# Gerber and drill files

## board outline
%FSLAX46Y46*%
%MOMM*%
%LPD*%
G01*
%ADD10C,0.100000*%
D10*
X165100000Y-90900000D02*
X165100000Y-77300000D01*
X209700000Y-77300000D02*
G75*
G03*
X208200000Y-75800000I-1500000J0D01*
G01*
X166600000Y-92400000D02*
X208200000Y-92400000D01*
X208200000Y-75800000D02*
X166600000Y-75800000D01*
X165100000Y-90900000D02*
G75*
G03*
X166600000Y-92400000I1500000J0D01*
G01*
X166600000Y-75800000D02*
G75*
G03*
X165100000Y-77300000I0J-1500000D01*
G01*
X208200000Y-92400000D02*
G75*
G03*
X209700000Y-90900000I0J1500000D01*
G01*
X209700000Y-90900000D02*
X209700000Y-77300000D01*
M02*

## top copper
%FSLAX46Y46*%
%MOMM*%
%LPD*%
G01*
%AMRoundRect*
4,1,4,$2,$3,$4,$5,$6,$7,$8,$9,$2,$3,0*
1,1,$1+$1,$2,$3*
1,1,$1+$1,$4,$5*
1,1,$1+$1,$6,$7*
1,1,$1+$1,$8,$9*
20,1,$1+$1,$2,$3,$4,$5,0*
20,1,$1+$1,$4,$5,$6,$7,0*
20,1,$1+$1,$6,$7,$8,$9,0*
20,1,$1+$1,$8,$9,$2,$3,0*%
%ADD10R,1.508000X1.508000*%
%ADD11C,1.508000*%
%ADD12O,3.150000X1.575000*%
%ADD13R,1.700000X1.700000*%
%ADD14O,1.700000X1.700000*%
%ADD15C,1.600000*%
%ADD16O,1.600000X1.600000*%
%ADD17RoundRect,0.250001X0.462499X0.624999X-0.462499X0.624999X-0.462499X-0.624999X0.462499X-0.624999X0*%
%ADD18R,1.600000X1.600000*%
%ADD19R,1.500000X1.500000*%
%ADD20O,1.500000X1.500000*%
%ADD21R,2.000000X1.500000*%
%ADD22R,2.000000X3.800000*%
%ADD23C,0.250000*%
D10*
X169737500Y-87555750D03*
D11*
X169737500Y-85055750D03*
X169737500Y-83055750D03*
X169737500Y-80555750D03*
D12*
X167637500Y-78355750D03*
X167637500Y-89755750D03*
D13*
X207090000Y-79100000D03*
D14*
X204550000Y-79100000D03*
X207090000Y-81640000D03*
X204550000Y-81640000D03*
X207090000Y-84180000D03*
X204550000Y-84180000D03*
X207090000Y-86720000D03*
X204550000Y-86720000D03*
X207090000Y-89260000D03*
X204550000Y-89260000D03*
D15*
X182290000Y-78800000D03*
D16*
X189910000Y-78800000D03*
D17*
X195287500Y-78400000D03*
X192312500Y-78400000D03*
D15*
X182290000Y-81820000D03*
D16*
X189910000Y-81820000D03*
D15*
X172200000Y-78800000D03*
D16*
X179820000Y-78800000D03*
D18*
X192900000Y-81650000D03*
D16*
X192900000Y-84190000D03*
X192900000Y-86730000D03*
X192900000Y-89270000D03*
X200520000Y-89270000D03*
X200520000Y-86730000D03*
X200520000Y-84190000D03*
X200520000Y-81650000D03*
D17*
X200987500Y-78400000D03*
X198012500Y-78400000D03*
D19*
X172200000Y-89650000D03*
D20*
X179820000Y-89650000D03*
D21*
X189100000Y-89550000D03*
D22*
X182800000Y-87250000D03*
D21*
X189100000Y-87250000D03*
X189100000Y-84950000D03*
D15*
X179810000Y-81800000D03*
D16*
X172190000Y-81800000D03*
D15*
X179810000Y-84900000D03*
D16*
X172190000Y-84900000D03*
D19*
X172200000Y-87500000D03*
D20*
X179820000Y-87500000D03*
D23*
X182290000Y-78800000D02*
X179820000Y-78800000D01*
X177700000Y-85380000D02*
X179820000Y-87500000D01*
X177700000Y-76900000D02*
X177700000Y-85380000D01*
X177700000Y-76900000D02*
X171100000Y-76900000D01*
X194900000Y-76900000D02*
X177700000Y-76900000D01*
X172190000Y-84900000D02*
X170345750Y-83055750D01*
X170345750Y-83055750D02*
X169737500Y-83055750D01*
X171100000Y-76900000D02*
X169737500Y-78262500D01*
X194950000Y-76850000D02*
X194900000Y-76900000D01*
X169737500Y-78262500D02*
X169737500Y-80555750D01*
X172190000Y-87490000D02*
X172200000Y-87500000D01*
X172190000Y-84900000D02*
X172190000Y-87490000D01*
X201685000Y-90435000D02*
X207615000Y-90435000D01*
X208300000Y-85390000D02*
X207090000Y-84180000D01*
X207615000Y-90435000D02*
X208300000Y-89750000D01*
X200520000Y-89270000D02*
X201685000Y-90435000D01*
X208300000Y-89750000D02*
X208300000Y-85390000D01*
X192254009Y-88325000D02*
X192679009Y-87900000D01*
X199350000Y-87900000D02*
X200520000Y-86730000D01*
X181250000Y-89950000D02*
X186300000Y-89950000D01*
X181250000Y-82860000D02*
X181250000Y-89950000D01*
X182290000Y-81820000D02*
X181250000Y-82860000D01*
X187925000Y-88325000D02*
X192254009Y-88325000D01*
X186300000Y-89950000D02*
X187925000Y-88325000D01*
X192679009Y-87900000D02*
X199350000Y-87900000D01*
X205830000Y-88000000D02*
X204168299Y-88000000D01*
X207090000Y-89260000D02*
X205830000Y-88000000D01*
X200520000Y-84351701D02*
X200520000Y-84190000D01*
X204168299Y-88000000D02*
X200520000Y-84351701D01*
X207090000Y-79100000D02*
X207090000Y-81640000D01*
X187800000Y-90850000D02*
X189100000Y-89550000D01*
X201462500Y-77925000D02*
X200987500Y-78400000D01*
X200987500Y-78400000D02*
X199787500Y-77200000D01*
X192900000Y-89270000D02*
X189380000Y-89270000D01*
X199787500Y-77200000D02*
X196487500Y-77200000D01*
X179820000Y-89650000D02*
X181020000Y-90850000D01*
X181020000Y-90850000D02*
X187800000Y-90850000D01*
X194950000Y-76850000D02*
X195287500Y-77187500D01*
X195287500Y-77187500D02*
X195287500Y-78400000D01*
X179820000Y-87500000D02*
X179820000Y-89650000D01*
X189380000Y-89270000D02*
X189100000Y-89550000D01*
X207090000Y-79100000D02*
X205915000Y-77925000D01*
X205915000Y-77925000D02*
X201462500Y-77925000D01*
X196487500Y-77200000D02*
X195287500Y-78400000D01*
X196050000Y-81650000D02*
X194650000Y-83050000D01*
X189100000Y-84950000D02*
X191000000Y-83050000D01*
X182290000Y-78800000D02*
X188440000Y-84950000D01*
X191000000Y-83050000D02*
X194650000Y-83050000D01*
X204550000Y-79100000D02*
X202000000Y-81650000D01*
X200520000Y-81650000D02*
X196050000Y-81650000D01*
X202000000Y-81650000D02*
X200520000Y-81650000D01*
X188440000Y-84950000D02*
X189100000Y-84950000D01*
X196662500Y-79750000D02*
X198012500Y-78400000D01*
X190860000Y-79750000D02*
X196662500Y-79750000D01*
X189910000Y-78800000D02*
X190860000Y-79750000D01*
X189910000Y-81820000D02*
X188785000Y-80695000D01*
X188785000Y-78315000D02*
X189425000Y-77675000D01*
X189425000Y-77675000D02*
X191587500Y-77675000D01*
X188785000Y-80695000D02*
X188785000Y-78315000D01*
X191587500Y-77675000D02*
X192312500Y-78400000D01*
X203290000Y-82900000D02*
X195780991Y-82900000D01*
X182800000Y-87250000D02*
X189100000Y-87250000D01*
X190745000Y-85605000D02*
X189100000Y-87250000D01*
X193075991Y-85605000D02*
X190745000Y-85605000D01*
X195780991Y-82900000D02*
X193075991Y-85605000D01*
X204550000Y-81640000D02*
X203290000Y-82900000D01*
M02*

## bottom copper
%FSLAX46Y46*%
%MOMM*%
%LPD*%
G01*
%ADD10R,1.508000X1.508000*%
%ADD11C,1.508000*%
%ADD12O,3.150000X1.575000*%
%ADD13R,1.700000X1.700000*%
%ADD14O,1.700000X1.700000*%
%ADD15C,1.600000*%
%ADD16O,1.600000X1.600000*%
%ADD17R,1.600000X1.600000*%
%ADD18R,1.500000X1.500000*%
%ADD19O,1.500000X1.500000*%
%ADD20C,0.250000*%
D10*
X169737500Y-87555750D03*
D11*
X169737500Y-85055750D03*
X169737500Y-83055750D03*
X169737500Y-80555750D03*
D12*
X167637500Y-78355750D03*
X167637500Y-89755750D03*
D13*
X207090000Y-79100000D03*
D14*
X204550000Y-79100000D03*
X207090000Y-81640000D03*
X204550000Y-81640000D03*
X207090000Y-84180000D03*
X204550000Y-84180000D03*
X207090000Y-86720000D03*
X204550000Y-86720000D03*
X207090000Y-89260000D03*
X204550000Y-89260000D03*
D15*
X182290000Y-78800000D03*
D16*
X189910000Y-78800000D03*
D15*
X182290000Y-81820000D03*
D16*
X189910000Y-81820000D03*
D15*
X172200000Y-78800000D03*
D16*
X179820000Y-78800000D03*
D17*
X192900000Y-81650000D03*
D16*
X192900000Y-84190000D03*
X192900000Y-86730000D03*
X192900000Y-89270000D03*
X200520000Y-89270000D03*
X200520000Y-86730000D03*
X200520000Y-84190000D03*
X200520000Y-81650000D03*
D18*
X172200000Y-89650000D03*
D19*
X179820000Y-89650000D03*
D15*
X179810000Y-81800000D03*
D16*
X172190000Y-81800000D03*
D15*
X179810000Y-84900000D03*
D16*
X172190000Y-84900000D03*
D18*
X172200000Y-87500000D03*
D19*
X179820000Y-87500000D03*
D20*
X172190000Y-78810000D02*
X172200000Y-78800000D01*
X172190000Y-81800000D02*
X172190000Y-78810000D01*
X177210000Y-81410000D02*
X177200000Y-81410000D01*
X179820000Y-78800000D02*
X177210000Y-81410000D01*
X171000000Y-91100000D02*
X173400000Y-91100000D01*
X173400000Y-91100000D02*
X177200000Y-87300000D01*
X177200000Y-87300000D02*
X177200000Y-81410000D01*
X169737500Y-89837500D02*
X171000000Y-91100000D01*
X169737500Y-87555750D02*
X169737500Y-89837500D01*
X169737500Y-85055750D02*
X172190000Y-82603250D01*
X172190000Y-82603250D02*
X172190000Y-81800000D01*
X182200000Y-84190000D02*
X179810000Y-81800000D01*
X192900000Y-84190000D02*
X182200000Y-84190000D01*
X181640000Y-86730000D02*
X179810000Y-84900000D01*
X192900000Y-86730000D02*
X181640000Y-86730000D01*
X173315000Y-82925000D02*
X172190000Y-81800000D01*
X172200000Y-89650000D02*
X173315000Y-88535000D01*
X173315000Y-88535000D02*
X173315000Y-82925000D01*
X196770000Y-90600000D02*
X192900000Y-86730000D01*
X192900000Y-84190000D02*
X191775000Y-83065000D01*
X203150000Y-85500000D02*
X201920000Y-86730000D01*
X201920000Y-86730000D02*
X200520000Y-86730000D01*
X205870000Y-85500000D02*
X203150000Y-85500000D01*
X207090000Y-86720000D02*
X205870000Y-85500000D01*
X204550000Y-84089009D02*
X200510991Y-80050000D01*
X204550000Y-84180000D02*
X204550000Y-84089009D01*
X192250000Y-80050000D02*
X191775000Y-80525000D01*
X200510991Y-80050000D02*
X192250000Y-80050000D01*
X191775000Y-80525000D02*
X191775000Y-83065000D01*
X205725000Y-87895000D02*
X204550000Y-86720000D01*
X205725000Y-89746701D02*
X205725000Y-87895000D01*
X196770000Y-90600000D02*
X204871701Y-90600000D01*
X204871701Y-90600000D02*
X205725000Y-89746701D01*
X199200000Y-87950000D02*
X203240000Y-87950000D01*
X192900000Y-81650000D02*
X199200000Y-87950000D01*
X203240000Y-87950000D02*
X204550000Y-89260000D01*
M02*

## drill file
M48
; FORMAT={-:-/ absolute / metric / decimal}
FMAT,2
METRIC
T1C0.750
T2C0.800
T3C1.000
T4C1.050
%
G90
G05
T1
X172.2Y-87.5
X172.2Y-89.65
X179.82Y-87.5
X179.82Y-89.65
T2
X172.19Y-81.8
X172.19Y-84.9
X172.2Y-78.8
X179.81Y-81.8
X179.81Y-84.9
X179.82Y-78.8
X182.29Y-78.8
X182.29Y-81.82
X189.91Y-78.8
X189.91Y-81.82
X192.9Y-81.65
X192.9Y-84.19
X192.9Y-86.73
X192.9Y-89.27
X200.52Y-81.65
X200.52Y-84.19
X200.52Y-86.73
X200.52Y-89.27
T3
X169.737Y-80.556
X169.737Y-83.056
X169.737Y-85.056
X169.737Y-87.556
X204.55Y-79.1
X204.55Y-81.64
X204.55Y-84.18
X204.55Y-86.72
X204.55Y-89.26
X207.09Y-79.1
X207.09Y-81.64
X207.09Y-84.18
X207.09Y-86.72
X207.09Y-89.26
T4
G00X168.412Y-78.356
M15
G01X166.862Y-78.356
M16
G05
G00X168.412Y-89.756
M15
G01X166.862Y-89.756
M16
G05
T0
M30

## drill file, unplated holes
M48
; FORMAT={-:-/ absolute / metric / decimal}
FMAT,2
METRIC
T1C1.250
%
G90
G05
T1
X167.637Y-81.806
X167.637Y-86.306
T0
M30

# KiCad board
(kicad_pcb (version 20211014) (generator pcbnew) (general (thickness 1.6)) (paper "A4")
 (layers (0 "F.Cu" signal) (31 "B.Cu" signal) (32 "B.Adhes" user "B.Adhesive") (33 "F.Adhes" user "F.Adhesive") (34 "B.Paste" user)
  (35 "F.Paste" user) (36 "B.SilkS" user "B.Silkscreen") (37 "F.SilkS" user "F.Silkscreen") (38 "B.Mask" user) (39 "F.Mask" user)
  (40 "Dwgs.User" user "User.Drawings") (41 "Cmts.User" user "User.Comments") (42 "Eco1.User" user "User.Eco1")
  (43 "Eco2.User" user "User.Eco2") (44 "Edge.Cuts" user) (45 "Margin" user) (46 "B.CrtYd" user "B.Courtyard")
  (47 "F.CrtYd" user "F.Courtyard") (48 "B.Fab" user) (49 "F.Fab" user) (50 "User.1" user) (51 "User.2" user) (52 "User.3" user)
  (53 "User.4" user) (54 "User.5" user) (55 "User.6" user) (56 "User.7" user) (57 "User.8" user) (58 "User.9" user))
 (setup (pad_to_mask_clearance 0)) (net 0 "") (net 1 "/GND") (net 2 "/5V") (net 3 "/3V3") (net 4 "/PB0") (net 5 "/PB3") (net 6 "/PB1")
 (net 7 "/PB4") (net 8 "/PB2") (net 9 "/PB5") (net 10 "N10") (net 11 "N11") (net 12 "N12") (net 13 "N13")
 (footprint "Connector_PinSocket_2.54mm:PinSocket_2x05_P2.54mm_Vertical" (layer "F.Cu") (at 207.09 79.1)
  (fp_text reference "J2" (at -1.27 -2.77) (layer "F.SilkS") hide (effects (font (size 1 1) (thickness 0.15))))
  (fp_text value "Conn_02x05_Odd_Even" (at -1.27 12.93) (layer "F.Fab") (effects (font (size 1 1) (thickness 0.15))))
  (pad "1" thru_hole rect (at 0 0) (size 1.7 1.7) (drill 1) (layers *.Cu *.Mask) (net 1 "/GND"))
  (pad "2" thru_hole oval (at -2.54 0) (size 1.7 1.7) (drill 1) (layers *.Cu *.Mask) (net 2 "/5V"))
  (pad "3" thru_hole oval (at 0 2.54) (size 1.7 1.7) (drill 1) (layers *.Cu *.Mask) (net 1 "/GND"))
  (pad "4" thru_hole oval (at -2.54 2.54) (size 1.7 1.7) (drill 1) (layers *.Cu *.Mask) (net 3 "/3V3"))
  (pad "5" thru_hole oval (at 0 5.08) (size 1.7 1.7) (drill 1) (layers *.Cu *.Mask) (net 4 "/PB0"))
  (pad "6" thru_hole oval (at -2.54 5.08) (size 1.7 1.7) (drill 1) (layers *.Cu *.Mask) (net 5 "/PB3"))
  (pad "7" thru_hole oval (at 0 7.62) (size 1.7 1.7) (drill 1) (layers *.Cu *.Mask) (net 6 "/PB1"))
  (pad "8" thru_hole oval (at -2.54 7.62) (size 1.7 1.7) (drill 1) (layers *.Cu *.Mask) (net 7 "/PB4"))
  (pad "9" thru_hole oval (at 0 10.16) (size 1.7 1.7) (drill 1) (layers *.Cu *.Mask) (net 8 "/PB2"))
  (pad "10" thru_hole oval (at -2.54 10.16) (size 1.7 1.7) (drill 1) (layers *.Cu *.Mask) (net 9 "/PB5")))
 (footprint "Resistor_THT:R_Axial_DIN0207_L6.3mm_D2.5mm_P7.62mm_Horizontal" (layer "F.Cu") (at 182.29 78.8)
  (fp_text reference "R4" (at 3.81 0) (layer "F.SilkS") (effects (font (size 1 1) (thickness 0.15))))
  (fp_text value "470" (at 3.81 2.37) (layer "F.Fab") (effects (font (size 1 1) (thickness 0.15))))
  (pad "1" thru_hole circle (at 0 0) (size 1.6 1.6) (drill 0.8) (layers *.Cu *.Mask) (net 2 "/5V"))
  (pad "2" thru_hole oval (at 7.62 0) (size 1.6 1.6) (drill 0.8) (layers *.Cu *.Mask) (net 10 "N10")))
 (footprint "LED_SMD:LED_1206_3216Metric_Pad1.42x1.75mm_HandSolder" (layer "F.Cu") (at 193.8 78.4 180)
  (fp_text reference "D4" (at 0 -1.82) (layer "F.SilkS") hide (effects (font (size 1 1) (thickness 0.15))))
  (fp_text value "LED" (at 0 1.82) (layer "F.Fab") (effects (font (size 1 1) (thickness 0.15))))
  (pad "1" smd roundrect (at -1.4875 0 180) (size 1.425 1.75) (layers "F.Cu" "F.Paste" "F.Mask") (roundrect_rratio 0.1754392982)
   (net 1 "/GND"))
  (pad "2" smd roundrect (at 1.4875 0 180) (size 1.425 1.75) (layers "F.Cu" "F.Paste" "F.Mask") (roundrect_rratio 0.1754392982)
   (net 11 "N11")))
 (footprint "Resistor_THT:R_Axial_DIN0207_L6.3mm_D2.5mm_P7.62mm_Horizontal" (layer "F.Cu") (at 182.29 81.82)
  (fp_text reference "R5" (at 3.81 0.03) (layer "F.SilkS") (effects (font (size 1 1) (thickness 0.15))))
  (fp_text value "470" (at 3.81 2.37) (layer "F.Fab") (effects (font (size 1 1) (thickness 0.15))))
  (pad "1" thru_hole circle (at 0 0) (size 1.6 1.6) (drill 0.8) (layers *.Cu *.Mask) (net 6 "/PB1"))
  (pad "2" thru_hole oval (at 7.62 0) (size 1.6 1.6) (drill 0.8) (layers *.Cu *.Mask) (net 11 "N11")))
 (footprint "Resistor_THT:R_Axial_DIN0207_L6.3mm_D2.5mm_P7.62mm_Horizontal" (layer "F.Cu") (at 172.2 78.8)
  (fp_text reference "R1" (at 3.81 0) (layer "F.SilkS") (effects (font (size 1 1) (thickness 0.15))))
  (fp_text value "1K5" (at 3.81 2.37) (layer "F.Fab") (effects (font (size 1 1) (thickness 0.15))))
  (pad "1" thru_hole circle (at 0 0) (size 1.6 1.6) (drill 0.8) (layers *.Cu *.Mask) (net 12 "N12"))
  (pad "2" thru_hole oval (at 7.62 0) (size 1.6 1.6) (drill 0.8) (layers *.Cu *.Mask) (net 2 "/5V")))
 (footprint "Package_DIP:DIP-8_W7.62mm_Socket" (layer "F.Cu") (at 192.9 81.65)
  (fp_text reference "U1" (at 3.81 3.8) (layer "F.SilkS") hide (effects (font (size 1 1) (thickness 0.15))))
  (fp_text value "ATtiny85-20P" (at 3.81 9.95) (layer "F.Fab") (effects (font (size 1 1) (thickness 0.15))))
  (pad "1" thru_hole rect (at 0 0) (size 1.6 1.6) (drill 0.8) (layers *.Cu *.Mask) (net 9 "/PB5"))
  (pad "2" thru_hole oval (at 0 2.54) (size 1.6 1.6) (drill 0.8) (layers *.Cu *.Mask) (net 5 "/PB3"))
  (pad "3" thru_hole oval (at 0 5.08) (size 1.6 1.6) (drill 0.8) (layers *.Cu *.Mask) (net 7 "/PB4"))
  (pad "4" thru_hole oval (at 0 7.62) (size 1.6 1.6) (drill 0.8) (layers *.Cu *.Mask) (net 1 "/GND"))
  (pad "5" thru_hole oval (at 7.62 7.62) (size 1.6 1.6) (drill 0.8) (layers *.Cu *.Mask) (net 4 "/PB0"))
  (pad "6" thru_hole oval (at 7.62 5.08) (size 1.6 1.6) (drill 0.8) (layers *.Cu *.Mask) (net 6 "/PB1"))
  (pad "7" thru_hole oval (at 7.62 2.54) (size 1.6 1.6) (drill 0.8) (layers *.Cu *.Mask) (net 8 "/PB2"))
  (pad "8" thru_hole oval (at 7.62 0) (size 1.6 1.6) (drill 0.8) (layers *.Cu *.Mask) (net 2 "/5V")))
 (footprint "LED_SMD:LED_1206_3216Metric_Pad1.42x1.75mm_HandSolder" (layer "F.Cu") (at 199.5 78.4 180)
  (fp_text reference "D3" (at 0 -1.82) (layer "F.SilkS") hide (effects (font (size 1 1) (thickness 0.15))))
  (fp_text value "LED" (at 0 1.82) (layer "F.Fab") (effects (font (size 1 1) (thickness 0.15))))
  (pad "1" smd roundrect (at -1.4875 0 180) (size 1.425 1.75) (layers "F.Cu" "F.Paste" "F.Mask") (roundrect_rratio 0.1754392982)
   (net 1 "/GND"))
  (pad "2" smd roundrect (at 1.4875 0 180) (size 1.425 1.75) (layers "F.Cu" "F.Paste" "F.Mask") (roundrect_rratio 0.1754392982)
   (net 10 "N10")))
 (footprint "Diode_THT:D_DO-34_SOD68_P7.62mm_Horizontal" (layer "F.Cu") (at 172.2 89.65)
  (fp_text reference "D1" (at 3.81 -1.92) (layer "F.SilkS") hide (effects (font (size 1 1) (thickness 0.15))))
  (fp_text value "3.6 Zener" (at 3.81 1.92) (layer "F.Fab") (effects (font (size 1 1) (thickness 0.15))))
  (pad "1" thru_hole rect (at 0 0) (size 1.5 1.5) (drill 0.75) (layers *.Cu *.Mask) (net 12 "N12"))
  (pad "2" thru_hole oval (at 7.62 0) (size 1.5 1.5) (drill 0.75) (layers *.Cu *.Mask) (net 1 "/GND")))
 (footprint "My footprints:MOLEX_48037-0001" (layer "F.Cu") (at 167.6375 84.05575 -90)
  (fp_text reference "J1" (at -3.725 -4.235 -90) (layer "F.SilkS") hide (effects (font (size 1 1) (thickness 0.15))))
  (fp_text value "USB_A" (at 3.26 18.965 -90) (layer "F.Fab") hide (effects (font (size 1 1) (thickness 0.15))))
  (pad "" np_thru_hole circle locked (at -2.25 0 270) (size 1.25 1.25) (drill 1.25) (layers *.Cu *.Mask))
  (pad "" np_thru_hole circle locked (at 2.25 0 270) (size 1.25 1.25) (drill 1.25) (layers *.Cu *.Mask))
  (pad "1" thru_hole rect locked (at 3.5 -2.1 270) (size 1.508 1.508) (drill 1) (layers *.Cu *.Mask) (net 2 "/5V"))
  (pad "2" thru_hole circle locked (at 1 -2.1 270) (size 1.508 1.508) (drill 1) (layers *.Cu *.Mask) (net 12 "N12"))
  (pad "3" thru_hole circle locked (at -1 -2.1 270) (size 1.508 1.508) (drill 1) (layers *.Cu *.Mask) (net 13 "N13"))
  (pad "4" thru_hole circle locked (at -3.5 -2.1 270) (size 1.508 1.508) (drill 1) (layers *.Cu *.Mask) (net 1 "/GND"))
  (pad "S1" thru_hole oval locked (at 5.7 0 270) (size 1.575 3.15) (drill oval 1.05 2.6) (layers *.Cu *.Mask))
  (pad "S2" thru_hole oval locked (at -5.7 0 270) (size 1.575 3.15) (drill oval 1.05 2.6) (layers *.Cu *.Mask)))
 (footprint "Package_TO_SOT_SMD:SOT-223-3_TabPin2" (layer "F.Cu") (at 185.95 87.25 180)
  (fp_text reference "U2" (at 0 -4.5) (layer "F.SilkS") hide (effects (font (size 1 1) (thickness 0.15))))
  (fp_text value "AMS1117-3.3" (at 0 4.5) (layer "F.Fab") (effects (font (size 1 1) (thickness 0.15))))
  (pad "1" smd rect (at -3.15 -2.3 180) (size 2 1.5) (layers "F.Cu" "F.Paste" "F.Mask") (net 1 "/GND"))
  (pad "2" smd rect (at 3.15 0 180) (size 2 3.8) (layers "F.Cu" "F.Paste" "F.Mask") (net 3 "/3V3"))
  (pad "2" smd rect (at -3.15 0 180) (size 2 1.5) (layers "F.Cu" "F.Paste" "F.Mask") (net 3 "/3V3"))
  (pad "3" smd rect (at -3.15 2.3 180) (size 2 1.5) (layers "F.Cu" "F.Paste" "F.Mask") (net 2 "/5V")))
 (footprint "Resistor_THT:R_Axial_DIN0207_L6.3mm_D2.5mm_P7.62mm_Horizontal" (layer "F.Cu") (at 179.81 81.8 180)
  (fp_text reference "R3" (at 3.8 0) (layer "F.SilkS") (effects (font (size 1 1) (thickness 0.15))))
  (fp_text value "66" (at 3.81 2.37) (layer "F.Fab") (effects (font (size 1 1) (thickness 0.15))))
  (pad "1" thru_hole circle (at 0 0 180) (size 1.6 1.6) (drill 0.8) (layers *.Cu *.Mask) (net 5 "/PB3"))
  (pad "2" thru_hole oval (at 7.62 0 180) (size 1.6 1.6) (drill 0.8) (layers *.Cu *.Mask) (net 12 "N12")))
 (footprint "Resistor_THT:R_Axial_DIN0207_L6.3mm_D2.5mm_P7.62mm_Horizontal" (layer "F.Cu") (at 179.81 84.9 180)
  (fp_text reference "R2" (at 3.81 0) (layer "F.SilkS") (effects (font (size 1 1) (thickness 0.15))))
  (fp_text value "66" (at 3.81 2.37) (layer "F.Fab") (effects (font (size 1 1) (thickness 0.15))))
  (pad "1" thru_hole circle (at 0 0 180) (size 1.6 1.6) (drill 0.8) (layers *.Cu *.Mask) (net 7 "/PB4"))
  (pad "2" thru_hole oval (at 7.62 0 180) (size 1.6 1.6) (drill 0.8) (layers *.Cu *.Mask) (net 13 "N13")))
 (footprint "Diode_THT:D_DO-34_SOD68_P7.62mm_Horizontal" (layer "F.Cu") (at 172.2 87.5)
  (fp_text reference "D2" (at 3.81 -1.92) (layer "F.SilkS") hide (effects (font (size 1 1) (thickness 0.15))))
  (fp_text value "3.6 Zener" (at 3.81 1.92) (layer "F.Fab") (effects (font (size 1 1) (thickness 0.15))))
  (pad "1" thru_hole rect (at 0 0) (size 1.5 1.5) (drill 0.75) (layers *.Cu *.Mask) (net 13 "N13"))
  (pad "2" thru_hole oval (at 7.62 0) (size 1.5 1.5) (drill 0.75) (layers *.Cu *.Mask) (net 1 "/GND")))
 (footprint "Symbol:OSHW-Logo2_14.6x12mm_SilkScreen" (layer "B.Cu") (at 186.1 86.8 180)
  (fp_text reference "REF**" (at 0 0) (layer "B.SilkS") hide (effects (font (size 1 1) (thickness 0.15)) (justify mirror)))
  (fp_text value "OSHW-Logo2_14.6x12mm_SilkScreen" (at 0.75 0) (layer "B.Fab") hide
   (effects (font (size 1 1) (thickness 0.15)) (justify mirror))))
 (gr_arc (start 208.2 75.8) (mid 209.26066 76.23934) (end 209.7 77.3) (layer "Edge.Cuts") (width 0.1))
 (gr_line (start 166.6 92.4) (end 208.2 92.4) (layer "Edge.Cuts") (width 0.1))
 (gr_line (start 208.2 75.8) (end 166.6 75.8) (layer "Edge.Cuts") (width 0.1))
 (gr_arc (start 166.6 92.4) (mid 165.53934 91.96066) (end 165.1 90.9) (layer "Edge.Cuts") (width 0.1))
 (gr_arc (start 165.1 77.3) (mid 165.53934 76.23934) (end 166.6 75.8) (layer "Edge.Cuts") (width 0.1))
 (gr_arc (start 209.7 90.9) (mid 209.26066 91.96066) (end 208.2 92.4) (layer "Edge.Cuts") (width 0.1))
 (gr_line (start 209.7 90.9) (end 209.7 77.3) (layer "Edge.Cuts") (width 0.1))
 (gr_line (start 165.1 90.9) (end 165.1 77.3) (layer "Edge.Cuts") (width 0.1))
 (segment (start 172.19 78.81) (end 172.2 78.8) (width 0.25) (layer "B.Cu") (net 12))
 (segment (start 173.315 88.535) (end 173.315 82.925) (width 0.25) (layer "B.Cu") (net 12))
 (segment (start 172.19 81.8) (end 172.19 78.81) (width 0.25) (layer "B.Cu") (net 12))
 (segment (start 173.315 82.925) (end 172.19 81.8) (width 0.25) (layer "B.Cu") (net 12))
 (segment (start 172.2 89.65) (end 173.315 88.535) (width 0.25) (layer "B.Cu") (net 12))
 (segment (start 169.7375 85.05575) (end 172.19 82.60325) (width 0.25) (layer "B.Cu") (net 12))
 (segment (start 172.19 82.60325) (end 172.19 81.8) (width 0.25) (layer "B.Cu") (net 12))
 (segment (start 170.34575 83.05575) (end 169.7375 83.05575) (width 0.25) (layer "F.Cu") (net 13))
 (segment (start 172.19 84.9) (end 170.34575 83.05575) (width 0.25) (layer "F.Cu") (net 13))
 (segment (start 172.19 87.49) (end 172.2 87.5) (width 0.25) (layer "F.Cu") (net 13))
 (segment (start 172.19 84.9) (end 172.19 87.49) (width 0.25) (layer "F.Cu") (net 13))
 (segment (start 201.685 90.435) (end 207.615 90.435) (width 0.25) (layer "F.Cu") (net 4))
 (segment (start 208.3 85.39) (end 207.09 84.18) (width 0.25) (layer "F.Cu") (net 4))
 (segment (start 207.615 90.435) (end 208.3 89.75) (width 0.25) (layer "F.Cu") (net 4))
 (segment (start 200.52 89.27) (end 201.685 90.435) (width 0.25) (layer "F.Cu") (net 4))
 (segment (start 208.3 89.75) (end 208.3 85.39) (width 0.25) (layer "F.Cu") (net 4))
 (segment (start 192.254009 88.325) (end 192.679009 87.9) (width 0.25) (layer "F.Cu") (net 6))
 (segment (start 199.35 87.9) (end 200.52 86.73) (width 0.25) (layer "F.Cu") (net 6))
 (segment (start 181.25 89.95) (end 186.3 89.95) (width 0.25) (layer "F.Cu") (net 6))
 (segment (start 181.25 82.86) (end 181.25 89.95) (width 0.25) (layer "F.Cu") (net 6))
 (segment (start 182.29 81.82) (end 181.25 82.86) (width 0.25) (layer "F.Cu") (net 6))
 (segment (start 187.925 88.325) (end 192.254009 88.325) (width 0.25) (layer "F.Cu") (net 6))
 (segment (start 186.3 89.95) (end 187.925 88.325) (width 0.25) (layer "F.Cu") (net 6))
 (segment (start 192.679009 87.9) (end 199.35 87.9) (width 0.25) (layer "F.Cu") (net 6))
 (segment (start 203.15 85.5) (end 201.92 86.73) (width 0.25) (layer "B.Cu") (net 6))
 (segment (start 201.92 86.73) (end 200.52 86.73) (width 0.25) (layer "B.Cu") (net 6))
 (segment (start 205.87 85.5) (end 203.15 85.5) (width 0.25) (layer "B.Cu") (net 6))
 (segment (start 207.09 86.72) (end 205.87 85.5) (width 0.25) (layer "B.Cu") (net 6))
 (segment (start 205.83 88) (end 204.168299 88) (width 0.25) (layer "F.Cu") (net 8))
 (segment (start 207.09 89.26) (end 205.83 88) (width 0.25) (layer "F.Cu") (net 8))
 (segment (start 200.52 84.351701) (end 200.52 84.19) (width 0.25) (layer "F.Cu") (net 8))
 (segment (start 204.168299 88) (end 200.52 84.351701) (width 0.25) (layer "F.Cu") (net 8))
 (segment (start 192.9 84.19) (end 182.2 84.19) (width 0.25) (layer "B.Cu") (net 5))
 (segment (start 204.55 84.089009) (end 200.510991 80.05) (width 0.25) (layer "B.Cu") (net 5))
 (segment (start 192.9 84.19) (end 191.775 83.065) (width 0.25) (layer "B.Cu") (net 5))
 (segment (start 182.2 84.19) (end 179.81 81.8) (width 0.25) (layer "B.Cu") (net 5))
 (segment (start 204.55 84.18) (end 204.55 84.089009) (width 0.25) (layer "B.Cu") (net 5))
 (segment (start 192.25 80.05) (end 191.775 80.525) (width 0.25) (layer "B.Cu") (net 5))
 (segment (start 200.510991 80.05) (end 192.25 80.05) (width 0.25) (layer "B.Cu") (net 5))
 (segment (start 191.775 80.525) (end 191.775 83.065) (width 0.25) (layer "B.Cu") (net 5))
 (segment (start 196.77 90.6) (end 192.9 86.73) (width 0.25) (layer "B.Cu") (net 7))
 (segment (start 205.725 87.895) (end 204.55 86.72) (width 0.25) (layer "B.Cu") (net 7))
 (segment (start 205.725 89.746701) (end 205.725 87.895) (width 0.25) (layer "B.Cu") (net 7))
 (segment (start 181.64 86.73) (end 179.81 84.9) (width 0.25) (layer "B.Cu") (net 7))
 (segment (start 196.77 90.6) (end 204.871701 90.6) (width 0.25) (layer "B.Cu") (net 7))
 (segment (start 192.9 86.73) (end 181.64 86.73) (width 0.25) (layer "B.Cu") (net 7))
 (segment (start 204.871701 90.6) (end 205.725 89.746701) (width 0.25) (layer "B.Cu") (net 7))
 (segment (start 199.2 87.95) (end 203.24 87.95) (width 0.25) (layer "B.Cu") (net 9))
 (segment (start 192.9 81.65) (end 199.2 87.95) (width 0.25) (layer "B.Cu") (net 9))
 (segment (start 203.24 87.95) (end 204.55 89.26) (width 0.25) (layer "B.Cu") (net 9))
 (segment (start 207.09 79.1) (end 207.09 81.64) (width 0.25) (layer "F.Cu") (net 1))
 (segment (start 187.8 90.85) (end 189.1 89.55) (width 0.25) (layer "F.Cu") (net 1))
 (segment (start 201.4625 77.925) (end 200.9875 78.4) (width 0.25) (layer "F.Cu") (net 1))
 (segment (start 177.7 76.9) (end 171.1 76.9) (width 0.25) (layer "F.Cu") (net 1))
 (segment (start 200.9875 78.4) (end 199.7875 77.2) (width 0.25) (layer "F.Cu") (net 1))
 (segment (start 194.95 76.85) (end 194.9 76.9) (width 0.25) (layer "F.Cu") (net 1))
 (segment (start 192.9 89.27) (end 189.38 89.27) (width 0.25) (layer "F.Cu") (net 1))
 (segment (start 199.7875 77.2) (end 196.4875 77.2) (width 0.25) (layer "F.Cu") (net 1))
 (segment (start 179.82 89.65) (end 181.02 90.85) (width 0.25) (layer "F.Cu") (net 1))
 (segment (start 181.02 90.85) (end 187.8 90.85) (width 0.25) (layer "F.Cu") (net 1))
 (segment (start 171.1 76.9) (end 169.7375 78.2625) (width 0.25) (layer "F.Cu") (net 1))
 (segment (start 194.95 76.85) (end 195.2875 77.1875) (width 0.25) (layer "F.Cu") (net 1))
 (segment (start 195.2875 77.1875) (end 195.2875 78.4) (width 0.25) (layer "F.Cu") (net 1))
 (segment (start 179.82 87.5) (end 179.82 89.65) (width 0.25) (layer "F.Cu") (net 1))
 (segment (start 177.7 76.9) (end 177.7 85.38) (width 0.25) (layer "F.Cu") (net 1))
 (segment (start 189.38 89.27) (end 189.1 89.55) (width 0.25) (layer "F.Cu") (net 1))
 (segment (start 177.7 85.38) (end 179.82 87.5) (width 0.25) (layer "F.Cu") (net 1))
 (segment (start 207.09 79.1) (end 205.915 77.925) (width 0.25) (layer "F.Cu") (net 1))
 (segment (start 194.9 76.9) (end 177.7 76.9) (width 0.25) (layer "F.Cu") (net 1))
 (segment (start 205.915 77.925) (end 201.4625 77.925) (width 0.25) (layer "F.Cu") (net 1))
 (segment (start 169.7375 78.2625) (end 169.7375 80.55575) (width 0.25) (layer "F.Cu") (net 1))
 (segment (start 196.4875 77.2) (end 195.2875 78.4) (width 0.25) (layer "F.Cu") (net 1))
 (segment (start 196.05 81.65) (end 194.65 83.05) (width 0.25) (layer "F.Cu") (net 2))
 (segment (start 189.1 84.95) (end 191 83.05) (width 0.25) (layer "F.Cu") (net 2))
 (segment (start 182.29 78.8) (end 179.82 78.8) (width 0.25) (layer "F.Cu") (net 2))
 (segment (start 182.29 78.8) (end 188.44 84.95) (width 0.25) (layer "F.Cu") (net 2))
 (segment (start 191 83.05) (end 194.65 83.05) (width 0.25) (layer "F.Cu") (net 2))
 (segment (start 204.55 79.1) (end 202 81.65) (width 0.25) (layer "F.Cu") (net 2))
 (segment (start 200.52 81.65) (end 196.05 81.65) (width 0.25) (layer "F.Cu") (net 2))
 (segment (start 202 81.65) (end 200.52 81.65) (width 0.25) (layer "F.Cu") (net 2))
 (segment (start 188.44 84.95) (end 189.1 84.95) (width 0.25) (layer "F.Cu") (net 2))
 (segment (start 171 91.1) (end 173.4 91.1) (width 0.25) (layer "B.Cu") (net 2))
 (segment (start 177.2 87.3) (end 177.2 81.41) (width 0.25) (layer "B.Cu") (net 2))
 (segment (start 169.7375 87.55575) (end 169.7375 89.8375) (width 0.25) (layer "B.Cu") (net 2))
 (segment (start 173.4 91.1) (end 177.2 87.3) (width 0.25) (layer "B.Cu") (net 2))
 (segment (start 179.82 78.8) (end 177.21 81.41) (width 0.25) (layer "B.Cu") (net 2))
 (segment (start 169.7375 89.8375) (end 171 91.1) (width 0.25) (layer "B.Cu") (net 2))
 (segment (start 177.21 81.41) (end 177.2 81.41) (width 0.25) (layer "B.Cu") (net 2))
 (segment (start 196.6625 79.75) (end 198.0125 78.4) (width 0.25) (layer "F.Cu") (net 10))
 (segment (start 190.86 79.75) (end 196.6625 79.75) (width 0.25) (layer "F.Cu") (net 10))
 (segment (start 189.91 78.8) (end 190.86 79.75) (width 0.25) (layer "F.Cu") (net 10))
 (segment (start 189.91 81.82) (end 188.785 80.695) (width 0.25) (layer "F.Cu") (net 11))
 (segment (start 188.785 78.315) (end 189.425 77.675) (width 0.25) (layer "F.Cu") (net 11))
 (segment (start 189.425 77.675) (end 191.5875 77.675) (width 0.25) (layer "F.Cu") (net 11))
 (segment (start 188.785 80.695) (end 188.785 78.315) (width 0.25) (layer "F.Cu") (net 11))
 (segment (start 191.5875 77.675) (end 192.3125 78.4) (width 0.25) (layer "F.Cu") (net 11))
 (segment (start 203.29 82.9) (end 195.780991 82.9) (width 0.25) (layer "F.Cu") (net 3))
 (segment (start 182.8 87.25) (end 189.1 87.25) (width 0.25) (layer "F.Cu") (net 3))
 (segment (start 190.745 85.605) (end 189.1 87.25) (width 0.25) (layer "F.Cu") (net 3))
 (segment (start 193.075991 85.605) (end 190.745 85.605) (width 0.25) (layer "F.Cu") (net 3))
 (segment (start 195.780991 82.9) (end 193.075991 85.605) (width 0.25) (layer "F.Cu") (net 3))
 (segment (start 204.55 81.64) (end 203.29 82.9) (width 0.25) (layer "F.Cu") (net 3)))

